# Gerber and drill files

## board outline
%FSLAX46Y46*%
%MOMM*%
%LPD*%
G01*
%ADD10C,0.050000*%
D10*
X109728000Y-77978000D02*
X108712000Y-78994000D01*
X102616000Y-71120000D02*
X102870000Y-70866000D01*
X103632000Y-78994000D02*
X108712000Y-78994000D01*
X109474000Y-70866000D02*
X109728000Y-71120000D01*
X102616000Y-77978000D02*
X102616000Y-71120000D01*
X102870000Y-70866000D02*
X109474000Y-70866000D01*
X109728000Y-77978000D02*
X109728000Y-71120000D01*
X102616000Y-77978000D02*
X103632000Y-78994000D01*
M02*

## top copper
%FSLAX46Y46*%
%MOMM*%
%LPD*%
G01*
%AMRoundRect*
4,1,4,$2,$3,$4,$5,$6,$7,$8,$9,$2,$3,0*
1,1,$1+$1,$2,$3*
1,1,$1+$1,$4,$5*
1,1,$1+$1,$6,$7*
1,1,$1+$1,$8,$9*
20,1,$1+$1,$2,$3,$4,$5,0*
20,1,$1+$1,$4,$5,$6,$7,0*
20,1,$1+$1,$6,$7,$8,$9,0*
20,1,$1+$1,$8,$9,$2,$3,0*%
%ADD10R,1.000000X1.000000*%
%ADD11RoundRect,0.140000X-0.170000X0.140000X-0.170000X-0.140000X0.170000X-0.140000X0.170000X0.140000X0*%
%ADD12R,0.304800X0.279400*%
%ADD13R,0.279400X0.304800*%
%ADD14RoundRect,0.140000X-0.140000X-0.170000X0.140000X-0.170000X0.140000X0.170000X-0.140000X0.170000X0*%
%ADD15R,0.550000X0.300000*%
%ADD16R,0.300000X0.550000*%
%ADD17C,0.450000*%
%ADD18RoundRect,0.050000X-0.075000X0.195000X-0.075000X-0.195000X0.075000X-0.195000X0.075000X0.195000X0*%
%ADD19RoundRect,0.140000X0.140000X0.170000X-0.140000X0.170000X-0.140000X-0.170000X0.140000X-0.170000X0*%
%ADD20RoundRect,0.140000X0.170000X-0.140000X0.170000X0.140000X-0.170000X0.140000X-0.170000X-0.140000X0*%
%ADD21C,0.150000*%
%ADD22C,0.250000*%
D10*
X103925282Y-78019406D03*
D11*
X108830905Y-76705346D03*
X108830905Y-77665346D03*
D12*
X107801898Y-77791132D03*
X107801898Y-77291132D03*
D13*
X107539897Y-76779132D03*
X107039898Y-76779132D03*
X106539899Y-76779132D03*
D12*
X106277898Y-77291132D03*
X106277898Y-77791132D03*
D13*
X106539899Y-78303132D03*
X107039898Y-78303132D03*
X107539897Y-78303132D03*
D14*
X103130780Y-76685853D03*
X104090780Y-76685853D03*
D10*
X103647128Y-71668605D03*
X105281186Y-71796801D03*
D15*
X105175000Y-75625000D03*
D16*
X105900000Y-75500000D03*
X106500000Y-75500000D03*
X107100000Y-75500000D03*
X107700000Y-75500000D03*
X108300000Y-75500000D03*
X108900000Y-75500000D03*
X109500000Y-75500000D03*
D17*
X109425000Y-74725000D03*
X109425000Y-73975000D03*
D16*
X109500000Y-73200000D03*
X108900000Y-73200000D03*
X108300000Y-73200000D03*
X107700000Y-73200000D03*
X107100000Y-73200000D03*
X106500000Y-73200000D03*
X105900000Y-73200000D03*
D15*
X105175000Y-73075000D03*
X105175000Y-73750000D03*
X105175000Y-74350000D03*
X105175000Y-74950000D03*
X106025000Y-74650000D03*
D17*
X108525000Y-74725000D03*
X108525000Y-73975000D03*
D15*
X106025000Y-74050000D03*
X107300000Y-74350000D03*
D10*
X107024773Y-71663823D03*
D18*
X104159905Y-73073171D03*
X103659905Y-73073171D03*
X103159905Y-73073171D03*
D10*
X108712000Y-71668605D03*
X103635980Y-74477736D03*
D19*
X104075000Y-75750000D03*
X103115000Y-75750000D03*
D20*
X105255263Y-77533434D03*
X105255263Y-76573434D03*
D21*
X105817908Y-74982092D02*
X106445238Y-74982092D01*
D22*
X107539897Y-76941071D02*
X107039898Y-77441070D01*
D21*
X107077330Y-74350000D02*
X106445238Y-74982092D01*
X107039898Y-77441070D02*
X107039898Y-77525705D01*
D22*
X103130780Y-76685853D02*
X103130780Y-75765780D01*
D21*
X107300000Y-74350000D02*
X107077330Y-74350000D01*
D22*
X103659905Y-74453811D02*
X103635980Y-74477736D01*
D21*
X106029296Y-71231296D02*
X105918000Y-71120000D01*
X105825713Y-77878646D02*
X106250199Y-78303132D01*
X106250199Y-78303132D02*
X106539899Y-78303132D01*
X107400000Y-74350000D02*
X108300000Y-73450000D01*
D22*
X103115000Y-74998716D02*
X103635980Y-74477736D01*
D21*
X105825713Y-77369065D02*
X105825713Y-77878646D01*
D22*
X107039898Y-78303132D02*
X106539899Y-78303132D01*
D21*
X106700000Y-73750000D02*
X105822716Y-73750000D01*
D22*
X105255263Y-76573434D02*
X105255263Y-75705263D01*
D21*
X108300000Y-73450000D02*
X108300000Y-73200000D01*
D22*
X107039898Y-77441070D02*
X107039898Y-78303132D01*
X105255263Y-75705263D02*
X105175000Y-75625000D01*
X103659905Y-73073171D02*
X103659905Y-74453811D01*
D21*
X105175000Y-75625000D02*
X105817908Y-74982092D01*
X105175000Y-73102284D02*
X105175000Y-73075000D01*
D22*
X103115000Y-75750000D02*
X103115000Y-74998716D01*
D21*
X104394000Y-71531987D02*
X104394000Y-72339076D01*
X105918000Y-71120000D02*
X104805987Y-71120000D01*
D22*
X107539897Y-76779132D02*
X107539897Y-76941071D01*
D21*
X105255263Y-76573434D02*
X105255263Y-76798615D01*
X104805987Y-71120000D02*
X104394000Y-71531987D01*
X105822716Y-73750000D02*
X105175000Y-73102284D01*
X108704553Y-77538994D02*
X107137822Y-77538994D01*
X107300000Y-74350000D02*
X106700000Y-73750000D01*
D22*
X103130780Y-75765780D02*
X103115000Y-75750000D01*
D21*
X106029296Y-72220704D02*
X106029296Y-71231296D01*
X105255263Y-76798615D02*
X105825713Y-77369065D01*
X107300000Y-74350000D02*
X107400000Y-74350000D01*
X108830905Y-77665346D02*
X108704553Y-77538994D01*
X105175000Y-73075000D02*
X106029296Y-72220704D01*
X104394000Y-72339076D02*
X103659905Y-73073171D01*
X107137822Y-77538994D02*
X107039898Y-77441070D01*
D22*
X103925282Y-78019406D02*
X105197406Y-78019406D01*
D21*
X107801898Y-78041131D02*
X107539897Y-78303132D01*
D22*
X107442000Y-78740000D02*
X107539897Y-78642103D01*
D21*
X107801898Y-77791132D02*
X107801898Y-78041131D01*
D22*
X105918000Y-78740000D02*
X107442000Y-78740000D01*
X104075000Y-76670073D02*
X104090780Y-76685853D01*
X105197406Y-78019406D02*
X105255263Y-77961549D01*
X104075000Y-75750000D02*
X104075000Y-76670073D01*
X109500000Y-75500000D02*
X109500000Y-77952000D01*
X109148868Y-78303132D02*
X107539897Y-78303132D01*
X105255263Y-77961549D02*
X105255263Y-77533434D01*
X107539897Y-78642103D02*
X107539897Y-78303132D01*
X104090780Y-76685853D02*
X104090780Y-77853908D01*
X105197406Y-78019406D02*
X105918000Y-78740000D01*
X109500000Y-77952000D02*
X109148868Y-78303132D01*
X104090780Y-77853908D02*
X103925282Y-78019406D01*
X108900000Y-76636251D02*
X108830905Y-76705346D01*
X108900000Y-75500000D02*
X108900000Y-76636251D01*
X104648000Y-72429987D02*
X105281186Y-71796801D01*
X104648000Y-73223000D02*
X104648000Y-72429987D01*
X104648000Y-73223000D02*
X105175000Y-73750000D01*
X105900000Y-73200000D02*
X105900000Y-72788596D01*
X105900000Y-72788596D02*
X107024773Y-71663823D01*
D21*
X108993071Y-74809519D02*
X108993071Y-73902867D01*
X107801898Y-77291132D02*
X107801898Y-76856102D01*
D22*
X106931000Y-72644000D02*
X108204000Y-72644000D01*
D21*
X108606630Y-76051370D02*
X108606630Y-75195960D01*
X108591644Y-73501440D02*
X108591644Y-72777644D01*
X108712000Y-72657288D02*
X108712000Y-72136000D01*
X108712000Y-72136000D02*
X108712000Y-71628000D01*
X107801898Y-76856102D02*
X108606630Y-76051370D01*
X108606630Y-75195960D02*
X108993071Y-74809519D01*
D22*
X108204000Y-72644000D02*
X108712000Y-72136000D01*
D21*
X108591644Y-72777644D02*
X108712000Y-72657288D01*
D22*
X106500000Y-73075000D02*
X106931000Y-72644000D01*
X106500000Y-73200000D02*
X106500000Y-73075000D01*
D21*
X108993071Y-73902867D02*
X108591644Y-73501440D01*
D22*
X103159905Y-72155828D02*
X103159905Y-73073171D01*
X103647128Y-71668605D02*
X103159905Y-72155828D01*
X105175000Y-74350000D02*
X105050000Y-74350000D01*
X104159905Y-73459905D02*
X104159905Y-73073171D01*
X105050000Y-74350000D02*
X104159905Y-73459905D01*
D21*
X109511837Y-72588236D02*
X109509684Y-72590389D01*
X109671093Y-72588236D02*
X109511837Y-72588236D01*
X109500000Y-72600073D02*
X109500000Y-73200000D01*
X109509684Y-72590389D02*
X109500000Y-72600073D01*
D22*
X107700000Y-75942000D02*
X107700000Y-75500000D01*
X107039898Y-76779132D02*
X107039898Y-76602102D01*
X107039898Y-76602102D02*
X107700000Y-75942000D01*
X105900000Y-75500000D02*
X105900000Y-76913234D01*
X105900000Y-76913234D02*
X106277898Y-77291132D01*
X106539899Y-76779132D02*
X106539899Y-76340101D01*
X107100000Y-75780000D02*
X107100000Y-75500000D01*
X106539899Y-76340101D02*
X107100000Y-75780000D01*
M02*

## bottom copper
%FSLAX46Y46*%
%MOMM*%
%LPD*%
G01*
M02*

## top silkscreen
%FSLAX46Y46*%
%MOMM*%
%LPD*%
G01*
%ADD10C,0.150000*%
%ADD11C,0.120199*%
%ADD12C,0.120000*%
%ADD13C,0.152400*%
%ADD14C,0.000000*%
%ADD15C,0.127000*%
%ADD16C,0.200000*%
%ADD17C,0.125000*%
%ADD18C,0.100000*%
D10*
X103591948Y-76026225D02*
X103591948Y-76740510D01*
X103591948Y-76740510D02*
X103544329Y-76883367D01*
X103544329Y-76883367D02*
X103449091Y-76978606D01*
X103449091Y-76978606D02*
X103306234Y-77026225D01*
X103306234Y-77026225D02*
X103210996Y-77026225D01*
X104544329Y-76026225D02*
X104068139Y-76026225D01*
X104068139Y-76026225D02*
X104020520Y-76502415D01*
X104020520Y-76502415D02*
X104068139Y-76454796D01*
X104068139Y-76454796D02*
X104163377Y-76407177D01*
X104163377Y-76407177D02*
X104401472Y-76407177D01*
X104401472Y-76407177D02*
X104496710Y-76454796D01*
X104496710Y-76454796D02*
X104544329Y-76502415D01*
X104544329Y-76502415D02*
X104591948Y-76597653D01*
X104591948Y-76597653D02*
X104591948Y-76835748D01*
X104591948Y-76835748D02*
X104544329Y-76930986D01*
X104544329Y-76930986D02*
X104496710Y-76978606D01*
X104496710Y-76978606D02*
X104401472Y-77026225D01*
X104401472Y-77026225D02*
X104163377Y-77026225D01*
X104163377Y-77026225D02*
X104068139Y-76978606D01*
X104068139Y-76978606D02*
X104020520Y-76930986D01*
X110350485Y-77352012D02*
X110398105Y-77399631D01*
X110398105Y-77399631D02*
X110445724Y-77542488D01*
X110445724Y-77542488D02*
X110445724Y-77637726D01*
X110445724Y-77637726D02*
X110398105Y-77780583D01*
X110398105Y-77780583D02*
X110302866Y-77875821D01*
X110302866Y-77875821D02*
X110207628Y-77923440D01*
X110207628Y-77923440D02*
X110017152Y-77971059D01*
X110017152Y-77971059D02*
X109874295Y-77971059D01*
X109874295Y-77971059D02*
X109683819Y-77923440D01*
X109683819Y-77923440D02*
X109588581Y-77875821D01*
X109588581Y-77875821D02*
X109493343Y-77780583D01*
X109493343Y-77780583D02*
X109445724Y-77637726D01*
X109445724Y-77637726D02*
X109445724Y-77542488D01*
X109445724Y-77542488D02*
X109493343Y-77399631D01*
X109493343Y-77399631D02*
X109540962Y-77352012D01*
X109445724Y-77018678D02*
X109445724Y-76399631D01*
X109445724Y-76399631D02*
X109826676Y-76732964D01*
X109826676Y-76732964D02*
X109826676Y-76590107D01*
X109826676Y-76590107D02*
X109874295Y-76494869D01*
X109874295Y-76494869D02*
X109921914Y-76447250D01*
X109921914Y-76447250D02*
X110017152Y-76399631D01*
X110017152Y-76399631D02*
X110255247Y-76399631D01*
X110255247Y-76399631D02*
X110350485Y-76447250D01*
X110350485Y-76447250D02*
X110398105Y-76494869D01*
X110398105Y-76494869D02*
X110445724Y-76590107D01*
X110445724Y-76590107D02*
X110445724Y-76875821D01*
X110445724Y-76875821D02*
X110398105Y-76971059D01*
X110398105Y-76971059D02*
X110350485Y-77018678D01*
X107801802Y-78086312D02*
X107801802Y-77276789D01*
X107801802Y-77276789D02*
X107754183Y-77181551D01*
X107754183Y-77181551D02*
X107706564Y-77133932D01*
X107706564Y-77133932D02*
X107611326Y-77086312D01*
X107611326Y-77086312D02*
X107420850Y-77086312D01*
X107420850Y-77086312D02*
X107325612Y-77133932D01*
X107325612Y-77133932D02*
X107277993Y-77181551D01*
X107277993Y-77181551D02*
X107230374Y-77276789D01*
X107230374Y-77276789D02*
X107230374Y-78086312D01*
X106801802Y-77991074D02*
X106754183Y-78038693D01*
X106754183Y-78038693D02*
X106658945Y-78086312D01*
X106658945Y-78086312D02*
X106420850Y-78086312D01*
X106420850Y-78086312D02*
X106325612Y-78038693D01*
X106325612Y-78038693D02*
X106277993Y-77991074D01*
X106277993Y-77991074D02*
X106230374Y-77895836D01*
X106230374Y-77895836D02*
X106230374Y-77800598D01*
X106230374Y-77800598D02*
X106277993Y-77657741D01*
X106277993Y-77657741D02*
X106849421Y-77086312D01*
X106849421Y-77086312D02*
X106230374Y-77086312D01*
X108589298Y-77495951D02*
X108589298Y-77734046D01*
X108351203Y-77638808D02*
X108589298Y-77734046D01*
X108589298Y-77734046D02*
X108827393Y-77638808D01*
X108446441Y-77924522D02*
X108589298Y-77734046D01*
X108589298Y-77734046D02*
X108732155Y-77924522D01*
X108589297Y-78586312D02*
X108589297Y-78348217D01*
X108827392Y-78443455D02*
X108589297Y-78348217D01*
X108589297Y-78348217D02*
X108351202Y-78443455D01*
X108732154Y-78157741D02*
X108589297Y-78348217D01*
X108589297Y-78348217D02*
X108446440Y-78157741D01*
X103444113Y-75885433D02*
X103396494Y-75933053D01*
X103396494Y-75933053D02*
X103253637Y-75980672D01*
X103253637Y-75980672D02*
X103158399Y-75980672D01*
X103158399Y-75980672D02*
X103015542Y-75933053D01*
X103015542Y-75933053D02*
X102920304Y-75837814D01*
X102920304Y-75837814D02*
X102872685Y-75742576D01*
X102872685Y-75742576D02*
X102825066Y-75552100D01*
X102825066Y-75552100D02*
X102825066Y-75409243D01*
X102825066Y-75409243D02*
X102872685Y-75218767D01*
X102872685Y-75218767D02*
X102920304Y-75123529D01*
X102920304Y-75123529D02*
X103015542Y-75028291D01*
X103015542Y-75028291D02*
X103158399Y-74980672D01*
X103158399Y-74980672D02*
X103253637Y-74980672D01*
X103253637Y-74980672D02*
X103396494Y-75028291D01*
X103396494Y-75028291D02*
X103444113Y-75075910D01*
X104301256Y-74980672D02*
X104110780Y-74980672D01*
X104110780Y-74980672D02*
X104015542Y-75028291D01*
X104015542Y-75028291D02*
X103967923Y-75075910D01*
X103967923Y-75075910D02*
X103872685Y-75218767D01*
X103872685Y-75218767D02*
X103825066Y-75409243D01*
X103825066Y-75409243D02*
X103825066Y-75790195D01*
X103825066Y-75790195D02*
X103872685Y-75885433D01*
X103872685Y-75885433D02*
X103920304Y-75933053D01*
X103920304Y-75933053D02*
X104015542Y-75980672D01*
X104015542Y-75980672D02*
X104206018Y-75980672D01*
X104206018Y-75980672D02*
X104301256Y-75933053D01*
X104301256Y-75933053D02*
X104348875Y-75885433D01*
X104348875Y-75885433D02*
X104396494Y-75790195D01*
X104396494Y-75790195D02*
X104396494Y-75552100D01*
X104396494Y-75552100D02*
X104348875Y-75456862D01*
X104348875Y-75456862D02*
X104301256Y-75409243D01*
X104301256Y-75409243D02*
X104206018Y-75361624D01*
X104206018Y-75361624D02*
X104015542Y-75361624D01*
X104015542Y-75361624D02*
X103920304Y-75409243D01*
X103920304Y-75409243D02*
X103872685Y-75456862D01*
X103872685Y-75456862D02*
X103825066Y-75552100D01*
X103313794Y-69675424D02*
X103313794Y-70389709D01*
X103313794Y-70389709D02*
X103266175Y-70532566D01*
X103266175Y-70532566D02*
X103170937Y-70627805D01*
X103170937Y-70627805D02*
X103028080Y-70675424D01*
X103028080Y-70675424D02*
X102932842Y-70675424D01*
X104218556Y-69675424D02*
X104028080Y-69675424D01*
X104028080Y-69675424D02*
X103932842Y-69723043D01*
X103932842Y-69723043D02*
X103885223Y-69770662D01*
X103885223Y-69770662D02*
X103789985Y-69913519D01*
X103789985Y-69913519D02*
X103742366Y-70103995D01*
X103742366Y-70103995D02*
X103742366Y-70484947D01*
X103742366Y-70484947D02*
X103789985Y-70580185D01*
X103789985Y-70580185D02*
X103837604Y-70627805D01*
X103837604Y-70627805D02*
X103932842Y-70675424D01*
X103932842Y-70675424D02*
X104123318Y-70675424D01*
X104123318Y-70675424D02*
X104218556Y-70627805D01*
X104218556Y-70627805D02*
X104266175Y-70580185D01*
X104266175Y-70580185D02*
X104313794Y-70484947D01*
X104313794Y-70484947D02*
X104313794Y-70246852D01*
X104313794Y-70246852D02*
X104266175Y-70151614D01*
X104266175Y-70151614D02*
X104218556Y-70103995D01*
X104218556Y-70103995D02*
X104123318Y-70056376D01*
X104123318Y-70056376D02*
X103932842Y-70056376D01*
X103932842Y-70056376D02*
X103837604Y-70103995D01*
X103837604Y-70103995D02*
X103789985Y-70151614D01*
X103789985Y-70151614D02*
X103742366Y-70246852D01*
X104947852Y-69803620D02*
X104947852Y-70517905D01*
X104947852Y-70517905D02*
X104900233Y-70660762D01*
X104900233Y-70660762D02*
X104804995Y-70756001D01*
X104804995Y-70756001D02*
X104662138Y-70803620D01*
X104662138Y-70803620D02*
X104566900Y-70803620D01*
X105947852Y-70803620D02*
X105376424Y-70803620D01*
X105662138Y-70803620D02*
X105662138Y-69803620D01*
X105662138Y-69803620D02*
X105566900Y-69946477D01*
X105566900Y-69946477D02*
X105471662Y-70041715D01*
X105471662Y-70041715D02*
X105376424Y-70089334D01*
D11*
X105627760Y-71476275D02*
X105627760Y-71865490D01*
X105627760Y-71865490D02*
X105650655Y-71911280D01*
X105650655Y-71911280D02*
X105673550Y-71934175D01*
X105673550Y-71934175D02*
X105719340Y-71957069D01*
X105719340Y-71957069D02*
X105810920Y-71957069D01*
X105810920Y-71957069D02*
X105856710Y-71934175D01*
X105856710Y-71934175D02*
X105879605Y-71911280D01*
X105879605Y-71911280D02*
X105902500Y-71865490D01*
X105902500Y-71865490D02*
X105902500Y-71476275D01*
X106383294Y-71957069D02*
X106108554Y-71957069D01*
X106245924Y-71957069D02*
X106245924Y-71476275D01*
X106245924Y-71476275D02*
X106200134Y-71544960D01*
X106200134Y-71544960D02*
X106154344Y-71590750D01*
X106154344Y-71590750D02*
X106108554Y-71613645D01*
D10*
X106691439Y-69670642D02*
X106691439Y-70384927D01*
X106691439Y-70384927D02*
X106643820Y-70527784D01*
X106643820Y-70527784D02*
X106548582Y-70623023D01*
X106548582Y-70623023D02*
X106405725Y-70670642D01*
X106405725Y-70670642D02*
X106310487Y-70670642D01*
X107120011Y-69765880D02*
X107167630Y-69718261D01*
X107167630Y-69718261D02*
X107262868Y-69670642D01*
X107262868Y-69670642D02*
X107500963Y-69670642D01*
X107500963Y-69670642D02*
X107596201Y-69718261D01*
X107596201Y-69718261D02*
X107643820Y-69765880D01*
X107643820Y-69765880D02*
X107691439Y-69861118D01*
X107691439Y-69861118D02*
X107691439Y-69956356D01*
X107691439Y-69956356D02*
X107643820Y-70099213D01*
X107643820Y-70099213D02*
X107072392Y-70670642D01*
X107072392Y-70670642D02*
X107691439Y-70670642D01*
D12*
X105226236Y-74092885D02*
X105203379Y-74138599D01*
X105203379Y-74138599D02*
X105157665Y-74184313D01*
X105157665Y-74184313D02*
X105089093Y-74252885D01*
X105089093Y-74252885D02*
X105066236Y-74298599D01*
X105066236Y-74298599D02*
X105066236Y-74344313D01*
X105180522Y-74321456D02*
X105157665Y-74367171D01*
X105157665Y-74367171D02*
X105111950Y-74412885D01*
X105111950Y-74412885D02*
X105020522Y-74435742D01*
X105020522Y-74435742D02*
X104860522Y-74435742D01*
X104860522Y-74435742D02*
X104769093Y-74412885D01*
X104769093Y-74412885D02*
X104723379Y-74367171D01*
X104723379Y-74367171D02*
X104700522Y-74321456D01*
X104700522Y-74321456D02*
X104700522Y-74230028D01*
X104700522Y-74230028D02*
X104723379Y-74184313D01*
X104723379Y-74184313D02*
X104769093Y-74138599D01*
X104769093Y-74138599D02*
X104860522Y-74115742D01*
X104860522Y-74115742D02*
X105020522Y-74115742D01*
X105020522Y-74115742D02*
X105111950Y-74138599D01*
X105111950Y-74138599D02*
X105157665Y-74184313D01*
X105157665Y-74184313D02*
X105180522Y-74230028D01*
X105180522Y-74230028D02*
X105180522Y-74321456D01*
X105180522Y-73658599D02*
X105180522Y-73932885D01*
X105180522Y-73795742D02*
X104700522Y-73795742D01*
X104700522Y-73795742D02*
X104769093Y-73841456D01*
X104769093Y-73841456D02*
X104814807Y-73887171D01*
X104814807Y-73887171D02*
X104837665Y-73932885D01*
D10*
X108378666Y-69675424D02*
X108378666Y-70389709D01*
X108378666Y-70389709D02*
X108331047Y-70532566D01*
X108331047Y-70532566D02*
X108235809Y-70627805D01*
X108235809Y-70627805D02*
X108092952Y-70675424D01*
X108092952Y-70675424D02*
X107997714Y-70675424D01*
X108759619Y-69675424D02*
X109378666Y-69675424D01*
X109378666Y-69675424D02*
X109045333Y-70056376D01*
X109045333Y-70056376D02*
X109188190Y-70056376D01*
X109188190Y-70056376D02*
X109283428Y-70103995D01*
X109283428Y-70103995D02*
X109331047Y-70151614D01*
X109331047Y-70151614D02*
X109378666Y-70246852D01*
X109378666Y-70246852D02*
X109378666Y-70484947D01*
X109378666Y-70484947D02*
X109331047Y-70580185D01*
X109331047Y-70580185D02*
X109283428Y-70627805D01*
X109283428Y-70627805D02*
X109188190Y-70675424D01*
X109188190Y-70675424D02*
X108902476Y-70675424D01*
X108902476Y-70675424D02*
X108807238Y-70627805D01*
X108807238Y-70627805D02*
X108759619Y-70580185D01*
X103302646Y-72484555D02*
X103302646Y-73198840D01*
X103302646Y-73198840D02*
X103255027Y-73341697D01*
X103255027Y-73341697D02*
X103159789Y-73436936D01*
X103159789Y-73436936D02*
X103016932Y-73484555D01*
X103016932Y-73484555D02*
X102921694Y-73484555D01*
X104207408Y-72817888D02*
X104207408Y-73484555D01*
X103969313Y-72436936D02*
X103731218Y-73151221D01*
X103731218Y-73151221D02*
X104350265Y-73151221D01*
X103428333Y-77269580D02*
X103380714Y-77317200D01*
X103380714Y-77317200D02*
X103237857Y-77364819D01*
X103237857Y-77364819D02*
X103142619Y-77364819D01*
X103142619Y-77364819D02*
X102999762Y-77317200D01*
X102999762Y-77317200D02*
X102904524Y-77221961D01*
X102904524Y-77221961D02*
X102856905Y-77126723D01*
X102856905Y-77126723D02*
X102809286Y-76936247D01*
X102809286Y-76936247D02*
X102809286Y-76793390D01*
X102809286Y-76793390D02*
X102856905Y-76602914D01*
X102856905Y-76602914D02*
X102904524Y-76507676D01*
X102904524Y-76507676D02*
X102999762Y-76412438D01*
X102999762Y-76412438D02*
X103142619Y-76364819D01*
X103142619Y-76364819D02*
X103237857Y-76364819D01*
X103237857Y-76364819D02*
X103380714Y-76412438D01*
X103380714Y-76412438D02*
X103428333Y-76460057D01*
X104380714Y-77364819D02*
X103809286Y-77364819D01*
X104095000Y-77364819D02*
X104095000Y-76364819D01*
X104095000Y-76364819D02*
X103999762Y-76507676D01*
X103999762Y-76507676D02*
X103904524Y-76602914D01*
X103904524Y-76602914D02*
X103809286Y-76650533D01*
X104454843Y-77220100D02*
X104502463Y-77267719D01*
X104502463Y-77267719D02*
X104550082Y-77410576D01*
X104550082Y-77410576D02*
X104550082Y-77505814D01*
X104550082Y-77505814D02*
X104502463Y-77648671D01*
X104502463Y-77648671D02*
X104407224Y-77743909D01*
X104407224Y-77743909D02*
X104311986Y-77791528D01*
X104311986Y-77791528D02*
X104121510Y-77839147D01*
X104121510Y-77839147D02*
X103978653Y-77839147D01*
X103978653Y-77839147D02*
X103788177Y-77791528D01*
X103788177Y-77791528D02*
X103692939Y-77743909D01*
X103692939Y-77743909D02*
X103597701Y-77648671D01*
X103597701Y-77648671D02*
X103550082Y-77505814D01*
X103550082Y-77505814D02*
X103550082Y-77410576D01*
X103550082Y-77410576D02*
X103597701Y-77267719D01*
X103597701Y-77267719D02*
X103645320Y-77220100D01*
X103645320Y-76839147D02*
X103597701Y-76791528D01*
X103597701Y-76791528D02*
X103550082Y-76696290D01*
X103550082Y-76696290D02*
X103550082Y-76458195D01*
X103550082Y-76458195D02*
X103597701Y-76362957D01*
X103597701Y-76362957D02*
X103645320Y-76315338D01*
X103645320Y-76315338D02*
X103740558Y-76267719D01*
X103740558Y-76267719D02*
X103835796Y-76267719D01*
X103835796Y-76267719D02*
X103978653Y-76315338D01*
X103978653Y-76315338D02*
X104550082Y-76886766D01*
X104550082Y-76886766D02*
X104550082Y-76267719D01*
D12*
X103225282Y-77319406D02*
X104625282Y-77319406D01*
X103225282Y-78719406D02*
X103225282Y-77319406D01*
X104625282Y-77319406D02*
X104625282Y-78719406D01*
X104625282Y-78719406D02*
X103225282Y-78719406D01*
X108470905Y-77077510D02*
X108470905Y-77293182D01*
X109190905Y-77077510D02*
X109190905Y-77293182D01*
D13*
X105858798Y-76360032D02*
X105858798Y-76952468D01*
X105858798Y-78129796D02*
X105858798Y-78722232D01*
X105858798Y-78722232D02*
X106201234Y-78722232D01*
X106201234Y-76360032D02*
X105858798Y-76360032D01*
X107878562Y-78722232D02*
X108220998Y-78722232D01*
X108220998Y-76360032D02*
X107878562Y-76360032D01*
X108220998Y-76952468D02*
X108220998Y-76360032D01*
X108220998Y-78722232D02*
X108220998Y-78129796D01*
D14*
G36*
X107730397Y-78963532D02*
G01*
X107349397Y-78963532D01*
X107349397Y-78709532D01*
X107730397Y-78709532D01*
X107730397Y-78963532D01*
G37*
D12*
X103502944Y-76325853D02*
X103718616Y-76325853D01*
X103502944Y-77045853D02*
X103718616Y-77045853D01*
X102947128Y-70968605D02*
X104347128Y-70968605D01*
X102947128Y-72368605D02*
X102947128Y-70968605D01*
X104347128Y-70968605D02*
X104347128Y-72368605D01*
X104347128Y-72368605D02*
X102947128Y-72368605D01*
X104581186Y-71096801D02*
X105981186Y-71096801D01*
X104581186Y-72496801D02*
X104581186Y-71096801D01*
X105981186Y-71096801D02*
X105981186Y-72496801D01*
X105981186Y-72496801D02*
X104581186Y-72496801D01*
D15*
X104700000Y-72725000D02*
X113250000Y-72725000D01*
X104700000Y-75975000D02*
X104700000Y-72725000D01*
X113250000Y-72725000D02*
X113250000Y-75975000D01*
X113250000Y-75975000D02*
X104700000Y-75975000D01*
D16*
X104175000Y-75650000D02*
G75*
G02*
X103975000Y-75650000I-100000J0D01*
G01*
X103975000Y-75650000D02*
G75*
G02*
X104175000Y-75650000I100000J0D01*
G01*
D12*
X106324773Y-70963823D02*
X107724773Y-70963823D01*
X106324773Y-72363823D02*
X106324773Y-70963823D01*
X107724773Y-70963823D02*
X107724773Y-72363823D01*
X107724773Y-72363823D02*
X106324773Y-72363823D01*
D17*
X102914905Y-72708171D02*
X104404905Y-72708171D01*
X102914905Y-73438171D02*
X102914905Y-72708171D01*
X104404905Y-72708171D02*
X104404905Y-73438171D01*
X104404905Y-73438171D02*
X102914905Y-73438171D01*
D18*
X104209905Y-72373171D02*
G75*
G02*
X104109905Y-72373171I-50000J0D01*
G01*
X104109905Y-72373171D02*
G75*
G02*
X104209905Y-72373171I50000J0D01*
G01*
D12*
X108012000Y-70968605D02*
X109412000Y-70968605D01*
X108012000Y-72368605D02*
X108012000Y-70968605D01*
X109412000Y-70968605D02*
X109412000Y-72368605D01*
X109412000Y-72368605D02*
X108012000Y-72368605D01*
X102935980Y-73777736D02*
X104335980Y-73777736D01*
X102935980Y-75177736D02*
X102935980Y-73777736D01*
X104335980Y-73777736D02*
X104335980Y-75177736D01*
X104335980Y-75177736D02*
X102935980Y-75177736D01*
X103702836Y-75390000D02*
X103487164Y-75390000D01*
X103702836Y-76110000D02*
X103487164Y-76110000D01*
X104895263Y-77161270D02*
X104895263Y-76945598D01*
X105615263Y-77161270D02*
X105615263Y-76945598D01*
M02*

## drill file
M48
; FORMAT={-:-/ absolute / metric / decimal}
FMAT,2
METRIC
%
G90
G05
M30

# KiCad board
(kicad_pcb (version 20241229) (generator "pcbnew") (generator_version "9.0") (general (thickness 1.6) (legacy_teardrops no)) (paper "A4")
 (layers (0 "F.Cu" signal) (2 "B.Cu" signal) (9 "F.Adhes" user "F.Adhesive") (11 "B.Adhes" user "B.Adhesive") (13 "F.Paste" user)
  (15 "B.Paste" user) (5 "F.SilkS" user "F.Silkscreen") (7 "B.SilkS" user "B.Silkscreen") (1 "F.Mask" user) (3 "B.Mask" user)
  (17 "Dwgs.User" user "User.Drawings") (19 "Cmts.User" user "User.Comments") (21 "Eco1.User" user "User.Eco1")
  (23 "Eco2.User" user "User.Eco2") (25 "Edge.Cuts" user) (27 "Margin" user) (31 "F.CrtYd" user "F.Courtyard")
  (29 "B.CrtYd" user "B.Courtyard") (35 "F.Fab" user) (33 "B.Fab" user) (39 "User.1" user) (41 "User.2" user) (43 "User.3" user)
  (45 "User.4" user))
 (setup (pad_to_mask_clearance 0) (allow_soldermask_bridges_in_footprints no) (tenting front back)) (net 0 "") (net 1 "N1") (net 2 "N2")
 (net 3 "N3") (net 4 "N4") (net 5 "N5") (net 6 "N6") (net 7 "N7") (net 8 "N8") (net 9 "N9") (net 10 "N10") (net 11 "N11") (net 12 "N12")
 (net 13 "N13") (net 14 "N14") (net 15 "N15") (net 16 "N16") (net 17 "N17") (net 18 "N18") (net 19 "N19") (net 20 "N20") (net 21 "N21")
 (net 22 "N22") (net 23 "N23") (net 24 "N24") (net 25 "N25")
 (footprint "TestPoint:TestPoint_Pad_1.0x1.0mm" (layer "F.Cu") (at 103.925282 78.019406)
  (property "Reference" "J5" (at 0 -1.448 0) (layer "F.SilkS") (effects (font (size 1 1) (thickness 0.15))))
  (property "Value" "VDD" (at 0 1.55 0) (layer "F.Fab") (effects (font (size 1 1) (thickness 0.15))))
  (fp_line (start -0.7 -0.7) (end 0.7 -0.7) (stroke (width 0.12) (type solid)) (layer "F.SilkS"))
  (fp_line (start -0.7 0.7) (end -0.7 -0.7) (stroke (width 0.12) (type solid)) (layer "F.SilkS"))
  (fp_line (start 0.7 -0.7) (end 0.7 0.7) (stroke (width 0.12) (type solid)) (layer "F.SilkS"))
  (fp_line (start 0.7 0.7) (end -0.7 0.7) (stroke (width 0.12) (type solid)) (layer "F.SilkS"))
  (pad "1" smd rect (at 0 0) (size 1 1) (layers "F.Cu" "F.Mask") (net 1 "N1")))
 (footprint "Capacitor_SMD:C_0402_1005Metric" (layer "F.Cu") (at 108.830905 77.185346 -90)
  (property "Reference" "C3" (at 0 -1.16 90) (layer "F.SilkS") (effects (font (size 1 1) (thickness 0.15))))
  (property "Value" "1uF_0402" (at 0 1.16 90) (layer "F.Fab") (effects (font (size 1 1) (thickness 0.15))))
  (fp_line (start -0.107836 0.36) (end 0.107836 0.36) (stroke (width 0.12) (type solid)) (layer "F.SilkS"))
  (fp_line (start -0.107836 -0.36) (end 0.107836 -0.36) (stroke (width 0.12) (type solid)) (layer "F.SilkS"))
  (pad "1" smd roundrect (at -0.48 0 270) (size 0.56 0.62) (layers "F.Cu" "F.Mask" "F.Paste") (roundrect_rratio 0.25) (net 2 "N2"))
  (pad "2" smd roundrect (at 0.48 0 270) (size 0.56 0.62) (layers "F.Cu" "F.Mask" "F.Paste") (roundrect_rratio 0.25) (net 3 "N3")))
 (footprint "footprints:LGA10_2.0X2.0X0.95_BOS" (layer "F.Cu") (at 107.039898 77.541132 180)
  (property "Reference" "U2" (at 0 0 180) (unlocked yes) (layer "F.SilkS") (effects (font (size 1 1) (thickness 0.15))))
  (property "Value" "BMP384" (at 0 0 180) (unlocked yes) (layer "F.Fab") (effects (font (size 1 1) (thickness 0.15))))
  (fp_line (start 1.1811 1.1811) (end 1.1811 0.588664) (stroke (width 0.1524) (type solid)) (layer "F.SilkS"))
  (fp_line (start 1.1811 -0.588664) (end 1.1811 -1.1811) (stroke (width 0.1524) (type solid)) (layer "F.SilkS"))
  (fp_line (start 1.1811 -1.1811) (end 0.838664 -1.1811) (stroke (width 0.1524) (type solid)) (layer "F.SilkS"))
  (fp_line (start 0.838664 1.1811) (end 1.1811 1.1811) (stroke (width 0.1524) (type solid)) (layer "F.SilkS"))
  (fp_line (start -0.838664 -1.1811) (end -1.1811 -1.1811) (stroke (width 0.1524) (type solid)) (layer "F.SilkS"))
  (fp_line (start -1.1811 1.1811) (end -0.838664 1.1811) (stroke (width 0.1524) (type solid)) (layer "F.SilkS"))
  (fp_line (start -1.1811 0.588664) (end -1.1811 1.1811) (stroke (width 0.1524) (type solid)) (layer "F.SilkS"))
  (fp_line (start -1.1811 -1.1811) (end -1.1811 -0.588664) (stroke (width 0.1524) (type solid)) (layer "F.SilkS"))
  (fp_poly
   (pts (xy -0.690499 -1.1684) (xy -0.690499 -1.4224) (xy -0.309499 -1.4224) (xy -0.309499 -1.1684)) (stroke (width 0) (type solid))
   (fill yes) (layer "F.SilkS"))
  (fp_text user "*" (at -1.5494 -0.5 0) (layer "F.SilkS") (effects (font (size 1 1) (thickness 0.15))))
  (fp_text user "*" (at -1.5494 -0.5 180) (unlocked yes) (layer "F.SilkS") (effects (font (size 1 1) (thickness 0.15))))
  (pad "1" smd rect (at -0.762 -0.25 270) (size 0.2794 0.3048) (layers "F.Cu" "F.Mask" "F.Paste") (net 1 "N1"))
  (pad "2" smd rect (at -0.762 0.25 270) (size 0.2794 0.3048) (layers "F.Cu" "F.Mask" "F.Paste") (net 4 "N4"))
  (pad "3" smd rect (at -0.499999 0.762 180) (size 0.2794 0.3048) (layers "F.Cu" "F.Mask" "F.Paste") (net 3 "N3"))
  (pad "4" smd rect (at 0 0.762 180) (size 0.2794 0.3048) (layers "F.Cu" "F.Mask" "F.Paste") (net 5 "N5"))
  (pad "5" smd rect (at 0.499999 0.762 180) (size 0.2794 0.3048) (layers "F.Cu" "F.Mask" "F.Paste") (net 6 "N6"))
  (pad "6" smd rect (at 0.762 0.25 270) (size 0.2794 0.3048) (layers "F.Cu" "F.Mask" "F.Paste") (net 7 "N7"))
  (pad "7" smd rect (at 0.762 -0.25 270) (size 0.2794 0.3048) (layers "F.Cu" "F.Mask" "F.Paste") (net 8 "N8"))
  (pad "8" smd rect (at 0.499999 -0.762 180) (size 0.2794 0.3048) (layers "F.Cu" "F.Mask" "F.Paste") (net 3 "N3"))
  (pad "9" smd rect (at 0 -0.762 180) (size 0.2794 0.3048) (layers "F.Cu" "F.Mask" "F.Paste") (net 3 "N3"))
  (pad "10" smd rect (at -0.499999 -0.762 180) (size 0.2794 0.3048) (layers "F.Cu" "F.Mask" "F.Paste") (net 1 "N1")))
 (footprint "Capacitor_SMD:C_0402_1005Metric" (layer "F.Cu") (at 103.61078 76.685853)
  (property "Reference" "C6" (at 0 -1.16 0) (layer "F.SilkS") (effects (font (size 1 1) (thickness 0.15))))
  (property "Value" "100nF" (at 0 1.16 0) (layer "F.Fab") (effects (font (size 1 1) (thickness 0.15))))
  (fp_line (start -0.107836 -0.36) (end 0.107836 -0.36) (stroke (width 0.12) (type solid)) (layer "F.SilkS"))
  (fp_line (start -0.107836 0.36) (end 0.107836 0.36) (stroke (width 0.12) (type solid)) (layer "F.SilkS"))
  (pad "1" smd roundrect (at -0.48 0) (size 0.56 0.62) (layers "F.Cu" "F.Mask" "F.Paste") (roundrect_rratio 0.25) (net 3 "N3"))
  (pad "2" smd roundrect (at 0.48 0) (size 0.56 0.62) (layers "F.Cu" "F.Mask" "F.Paste") (roundrect_rratio 0.25) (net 1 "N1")))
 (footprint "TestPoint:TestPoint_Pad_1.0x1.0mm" (layer "F.Cu") (at 103.647128 71.668605)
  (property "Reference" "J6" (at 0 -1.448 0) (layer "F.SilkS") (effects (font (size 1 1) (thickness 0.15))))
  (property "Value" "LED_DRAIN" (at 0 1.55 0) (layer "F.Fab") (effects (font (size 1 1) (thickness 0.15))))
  (fp_line (start -0.7 -0.7) (end 0.7 -0.7) (stroke (width 0.12) (type solid)) (layer "F.SilkS"))
  (fp_line (start -0.7 0.7) (end -0.7 -0.7) (stroke (width 0.12) (type solid)) (layer "F.SilkS"))
  (fp_line (start 0.7 -0.7) (end 0.7 0.7) (stroke (width 0.12) (type solid)) (layer "F.SilkS"))
  (fp_line (start 0.7 0.7) (end -0.7 0.7) (stroke (width 0.12) (type solid)) (layer "F.SilkS"))
  (pad "1" smd rect (at 0 0) (size 1 1) (layers "F.Cu" "F.Mask") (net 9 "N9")))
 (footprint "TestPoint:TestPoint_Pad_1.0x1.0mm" (layer "F.Cu") (at 105.281186 71.796801)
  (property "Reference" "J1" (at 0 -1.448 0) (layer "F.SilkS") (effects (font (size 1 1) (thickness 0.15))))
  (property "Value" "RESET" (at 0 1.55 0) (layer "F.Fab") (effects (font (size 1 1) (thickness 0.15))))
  (fp_line (start -0.7 -0.7) (end 0.7 -0.7) (stroke (width 0.12) (type solid)) (layer "F.SilkS"))
  (fp_line (start -0.7 0.7) (end -0.7 -0.7) (stroke (width 0.12) (type solid)) (layer "F.SilkS"))
  (fp_line (start 0.7 -0.7) (end 0.7 0.7) (stroke (width 0.12) (type solid)) (layer "F.SilkS"))
  (fp_line (start 0.7 0.7) (end -0.7 0.7) (stroke (width 0.12) (type solid)) (layer "F.SilkS"))
  (pad "1" smd rect (at 0 0) (size 1 1) (layers "F.Cu" "F.Mask") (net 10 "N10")))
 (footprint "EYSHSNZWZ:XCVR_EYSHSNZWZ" (layer "F.Cu") (at 108.975 74.35)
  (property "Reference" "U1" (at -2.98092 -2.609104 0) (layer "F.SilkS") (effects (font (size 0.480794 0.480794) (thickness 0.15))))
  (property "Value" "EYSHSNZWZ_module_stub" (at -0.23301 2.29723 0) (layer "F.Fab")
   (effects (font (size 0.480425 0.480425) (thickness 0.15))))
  (fp_line (start -4.275 -1.625) (end 4.275 -1.625) (stroke (width 0.127) (type solid)) (layer "F.SilkS"))
  (fp_line (start -4.275 1.625) (end -4.275 -1.625) (stroke (width 0.127) (type solid)) (layer "F.SilkS"))
  (fp_line (start 4.275 -1.625) (end 4.275 1.625) (stroke (width 0.127) (type solid)) (layer "F.SilkS"))
  (fp_line (start 4.275 1.625) (end -4.275 1.625) (stroke (width 0.127) (type solid)) (layer "F.SilkS"))
  (fp_circle (center -4.9 1.3) (end -4.8 1.3) (stroke (width 0.2) (type solid)) (fill no) (layer "F.SilkS"))
  (pad "1" smd rect (at -3.8 1.275) (size 0.55 0.3) (layers "F.Cu" "F.Mask") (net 3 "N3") (solder_mask_margin 0.102))
  (pad "2" smd rect (at -3.075 1.15) (size 0.3 0.55) (layers "F.Cu" "F.Mask") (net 7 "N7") (solder_mask_margin 0.102))
  (pad "3" smd rect (at -2.475 1.15) (size 0.3 0.55) (layers "F.Cu" "F.Mask") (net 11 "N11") (solder_mask_margin 0.102))
  (pad "4" smd rect (at -1.875 1.15) (size 0.3 0.55) (layers "F.Cu" "F.Mask") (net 6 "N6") (solder_mask_margin 0.102))
  (pad "5" smd rect (at -1.275 1.15) (size 0.3 0.55) (layers "F.Cu" "F.Mask") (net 5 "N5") (solder_mask_margin 0.102))
  (pad "6" smd rect (at -0.675 1.15) (size 0.3 0.55) (layers "F.Cu" "F.Mask") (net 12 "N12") (solder_mask_margin 0.102))
  (pad "7" smd rect (at -0.075 1.15) (size 0.3 0.55) (layers "F.Cu" "F.Mask") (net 2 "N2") (solder_mask_margin 0.102))
  (pad "8" smd rect (at 0.525 1.15) (size 0.3 0.55) (layers "F.Cu" "F.Mask") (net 1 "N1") (solder_mask_margin 0.102))
  (pad "9" smd circle (at 0.45 0.375) (size 0.45 0.45) (layers "F.Cu" "F.Mask") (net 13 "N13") (solder_mask_margin 0.102))
  (pad "10" smd circle (at 0.45 -0.375) (size 0.45 0.45) (layers "F.Cu" "F.Mask") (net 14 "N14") (solder_mask_margin 0.102))
  (pad "11" smd rect (at 0.525 -1.15) (size 0.3 0.55) (layers "F.Cu" "F.Mask") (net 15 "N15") (solder_mask_margin 0.102))
  (pad "12" smd rect (at -0.075 -1.15) (size 0.3 0.55) (layers "F.Cu" "F.Mask") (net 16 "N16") (solder_mask_margin 0.102))
  (pad "13" smd rect (at -0.675 -1.15) (size 0.3 0.55) (layers "F.Cu" "F.Mask") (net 3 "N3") (solder_mask_margin 0.102))
  (pad "14" smd rect (at -1.275 -1.15) (size 0.3 0.55) (layers "F.Cu" "F.Mask") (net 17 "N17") (solder_mask_margin 0.102))
  (pad "15" smd rect (at -1.875 -1.15) (size 0.3 0.55) (layers "F.Cu" "F.Mask") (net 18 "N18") (solder_mask_margin 0.102))
  (pad "16" smd rect (at -2.475 -1.15) (size 0.3 0.55) (layers "F.Cu" "F.Mask") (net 4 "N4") (solder_mask_margin 0.102))
  (pad "17" smd rect (at -3.075 -1.15) (size 0.3 0.55) (layers "F.Cu" "F.Mask") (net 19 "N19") (solder_mask_margin 0.102))
  (pad "18" smd rect (at -3.8 -1.275) (size 0.55 0.3) (layers "F.Cu" "F.Mask") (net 3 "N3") (solder_mask_margin 0.102))
  (pad "19" smd rect (at -3.8 -0.6) (size 0.55 0.3) (layers "F.Cu" "F.Mask") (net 10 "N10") (solder_mask_margin 0.102))
  (pad "20" smd rect (at -3.8 0) (size 0.55 0.3) (layers "F.Cu" "F.Mask") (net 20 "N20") (solder_mask_margin 0.102))
  (pad "21" smd rect (at -3.8 0.6) (size 0.55 0.3) (layers "F.Cu" "F.Mask") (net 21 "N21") (solder_mask_margin 0.102))
  (pad "22" smd rect (at -2.95 0.3) (size 0.55 0.3) (layers "F.Cu" "F.Mask") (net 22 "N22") (solder_mask_margin 0.102))
  (pad "23" smd circle (at -0.45 0.375) (size 0.45 0.45) (layers "F.Cu" "F.Mask") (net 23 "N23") (solder_mask_margin 0.102))
  (pad "24" smd circle (at -0.45 -0.375) (size 0.45 0.45) (layers "F.Cu" "F.Mask") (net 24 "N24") (solder_mask_margin 0.102))
  (pad "25" smd rect (at -2.95 -0.3) (size 0.55 0.3) (layers "F.Cu" "F.Mask") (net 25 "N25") (solder_mask_margin 0.102))
  (pad "26" smd rect (at -1.675 0) (size 0.55 0.3) (layers "F.Cu" "F.Mask") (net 3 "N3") (solder_mask_margin 0.102)))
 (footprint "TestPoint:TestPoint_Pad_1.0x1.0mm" (layer "F.Cu") (at 107.024773 71.663823)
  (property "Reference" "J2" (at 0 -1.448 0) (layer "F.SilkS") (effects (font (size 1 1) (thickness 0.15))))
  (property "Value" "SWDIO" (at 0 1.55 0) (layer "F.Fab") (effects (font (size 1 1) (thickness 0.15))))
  (fp_line (start -0.7 -0.7) (end 0.7 -0.7) (stroke (width 0.12) (type solid)) (layer "F.SilkS"))
  (fp_line (start -0.7 0.7) (end -0.7 -0.7) (stroke (width 0.12) (type solid)) (layer "F.SilkS"))
  (fp_line (start 0.7 -0.7) (end 0.7 0.7) (stroke (width 0.12) (type solid)) (layer "F.SilkS"))
  (fp_line (start 0.7 0.7) (end -0.7 0.7) (stroke (width 0.12) (type solid)) (layer "F.SilkS"))
  (pad "1" smd rect (at 0 0) (size 1 1) (layers "F.Cu" "F.Mask") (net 19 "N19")))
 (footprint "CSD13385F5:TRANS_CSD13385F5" (layer "F.Cu") (at 103.659905 73.073171 -90)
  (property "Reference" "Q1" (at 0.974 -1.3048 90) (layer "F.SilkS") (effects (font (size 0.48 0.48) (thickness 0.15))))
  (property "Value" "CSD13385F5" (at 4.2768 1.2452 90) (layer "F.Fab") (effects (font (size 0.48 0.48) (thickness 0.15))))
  (fp_line (start -0.365 0.745) (end -0.365 -0.745) (stroke (width 0.125) (type solid)) (layer "F.SilkS"))
  (fp_line (start 0.365 0.745) (end -0.365 0.745) (stroke (width 0.125) (type solid)) (layer "F.SilkS"))
  (fp_line (start -0.365 -0.745) (end 0.365 -0.745) (stroke (width 0.125) (type solid)) (layer "F.SilkS"))
  (fp_line (start 0.365 -0.745) (end 0.365 0.745) (stroke (width 0.125) (type solid)) (layer "F.SilkS"))
  (fp_circle (center -0.7 -0.5) (end -0.65 -0.5) (stroke (width 0.1) (type solid)) (fill no) (layer "F.SilkS"))
  (pad "1" smd roundrect (at 0 -0.5 270) (size 0.49 0.25) (layers "F.Cu") (roundrect_rratio 0.2) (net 20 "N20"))
  (pad "2" smd roundrect (at 0 0 270) (size 0.49 0.25) (layers "F.Cu") (roundrect_rratio 0.2) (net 3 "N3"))
  (pad "3" smd roundrect (at 0 0.5 270) (size 0.49 0.25) (layers "F.Cu") (roundrect_rratio 0.2) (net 9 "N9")))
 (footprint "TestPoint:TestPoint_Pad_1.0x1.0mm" (layer "F.Cu") (at 108.712 71.668605)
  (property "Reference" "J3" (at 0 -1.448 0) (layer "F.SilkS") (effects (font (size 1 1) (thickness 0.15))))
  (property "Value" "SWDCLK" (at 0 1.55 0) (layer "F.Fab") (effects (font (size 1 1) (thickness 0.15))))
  (fp_line (start -0.7 -0.7) (end 0.7 -0.7) (stroke (width 0.12) (type solid)) (layer "F.SilkS"))
  (fp_line (start -0.7 0.7) (end -0.7 -0.7) (stroke (width 0.12) (type solid)) (layer "F.SilkS"))
  (fp_line (start 0.7 -0.7) (end 0.7 0.7) (stroke (width 0.12) (type solid)) (layer "F.SilkS"))
  (fp_line (start 0.7 0.7) (end -0.7 0.7) (stroke (width 0.12) (type solid)) (layer "F.SilkS"))
  (pad "1" smd rect (at 0 0) (size 1 1) (layers "F.Cu" "F.Mask") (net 4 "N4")))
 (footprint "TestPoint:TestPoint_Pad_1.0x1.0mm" (layer "F.Cu") (at 103.63598 74.477736)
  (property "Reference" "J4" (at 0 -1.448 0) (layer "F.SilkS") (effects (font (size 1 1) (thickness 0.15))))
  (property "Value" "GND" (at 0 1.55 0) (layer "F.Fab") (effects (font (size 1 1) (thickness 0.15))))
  (fp_line (start -0.7 -0.7) (end 0.7 -0.7) (stroke (width 0.12) (type solid)) (layer "F.SilkS"))
  (fp_line (start -0.7 0.7) (end -0.7 -0.7) (stroke (width 0.12) (type solid)) (layer "F.SilkS"))
  (fp_line (start 0.7 -0.7) (end 0.7 0.7) (stroke (width 0.12) (type solid)) (layer "F.SilkS"))
  (fp_line (start 0.7 0.7) (end -0.7 0.7) (stroke (width 0.12) (type solid)) (layer "F.SilkS"))
  (pad "1" smd rect (at 0 0) (size 1 1) (layers "F.Cu" "F.Mask") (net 3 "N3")))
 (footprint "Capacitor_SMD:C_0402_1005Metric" (layer "F.Cu") (at 103.595 75.75 180)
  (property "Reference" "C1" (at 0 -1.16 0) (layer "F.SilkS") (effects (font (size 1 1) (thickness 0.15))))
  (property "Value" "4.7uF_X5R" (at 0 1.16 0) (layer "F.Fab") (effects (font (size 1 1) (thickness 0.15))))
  (fp_line (start -0.107836 0.36) (end 0.107836 0.36) (stroke (width 0.12) (type solid)) (layer "F.SilkS"))
  (fp_line (start -0.107836 -0.36) (end 0.107836 -0.36) (stroke (width 0.12) (type solid)) (layer "F.SilkS"))
  (pad "1" smd roundrect (at -0.48 0 180) (size 0.56 0.62) (layers "F.Cu" "F.Mask" "F.Paste") (roundrect_rratio 0.25) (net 1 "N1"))
  (pad "2" smd roundrect (at 0.48 0 180) (size 0.56 0.62) (layers "F.Cu" "F.Mask" "F.Paste") (roundrect_rratio 0.25) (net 3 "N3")))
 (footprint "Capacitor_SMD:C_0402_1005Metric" (layer "F.Cu") (at 105.255263 77.053434 90)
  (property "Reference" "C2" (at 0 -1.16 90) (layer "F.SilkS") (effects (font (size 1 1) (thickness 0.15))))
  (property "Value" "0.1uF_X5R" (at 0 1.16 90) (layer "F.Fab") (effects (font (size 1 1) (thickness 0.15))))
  (fp_line (start -0.107836 -0.36) (end 0.107836 -0.36) (stroke (width 0.12) (type solid)) (layer "F.SilkS"))
  (fp_line (start -0.107836 0.36) (end 0.107836 0.36) (stroke (width 0.12) (type solid)) (layer "F.SilkS"))
  (pad "1" smd roundrect (at -0.48 0 90) (size 0.56 0.62) (layers "F.Cu" "F.Mask" "F.Paste") (roundrect_rratio 0.25) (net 1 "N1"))
  (pad "2" smd roundrect (at 0.48 0 90) (size 0.56 0.62) (layers "F.Cu" "F.Mask" "F.Paste") (roundrect_rratio 0.25) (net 3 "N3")))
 (gr_line (start 109.728 77.978) (end 108.712 78.994) (stroke (width 0.05) (type default)) (layer "Edge.Cuts"))
 (gr_line (start 102.616 71.12) (end 102.87 70.866) (stroke (width 0.05) (type default)) (layer "Edge.Cuts"))
 (gr_line (start 103.632 78.994) (end 108.712 78.994) (stroke (width 0.05) (type default)) (layer "Edge.Cuts"))
 (gr_line (start 109.474 70.866) (end 109.728 71.12) (stroke (width 0.05) (type default)) (layer "Edge.Cuts"))
 (gr_line (start 102.616 77.978) (end 102.616 71.12) (stroke (width 0.05) (type default)) (layer "Edge.Cuts"))
 (gr_line (start 102.87 70.866) (end 109.474 70.866) (stroke (width 0.05) (type default)) (layer "Edge.Cuts"))
 (gr_line (start 109.728 77.978) (end 109.728 71.12) (stroke (width 0.05) (type default)) (layer "Edge.Cuts"))
 (gr_line (start 102.616 77.978) (end 103.632 78.994) (stroke (width 0.05) (type default)) (layer "Edge.Cuts"))
 (segment (start 105.817908 74.982092) (end 106.445238 74.982092) (width 0.15) (layer "F.Cu") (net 3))
 (segment (start 107.539897 76.941071) (end 107.039898 77.44107) (width 0.25) (layer "F.Cu") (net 3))
 (segment (start 107.07733 74.35) (end 106.445238 74.982092) (width 0.15) (layer "F.Cu") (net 3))
 (segment (start 107.039898 77.44107) (end 107.039898 77.525705) (width 0.15) (layer "F.Cu") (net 3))
 (segment (start 103.13078 76.685853) (end 103.13078 75.76578) (width 0.25) (layer "F.Cu") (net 3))
 (segment (start 107.3 74.35) (end 107.07733 74.35) (width 0.15) (layer "F.Cu") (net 3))
 (segment (start 103.659905 74.453811) (end 103.63598 74.477736) (width 0.25) (layer "F.Cu") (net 3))
 (segment (start 106.029296 71.231296) (end 105.918 71.12) (width 0.15) (layer "F.Cu") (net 3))
 (segment (start 105.825713 77.878646) (end 106.250199 78.303132) (width 0.15) (layer "F.Cu") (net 3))
 (segment (start 106.250199 78.303132) (end 106.539899 78.303132) (width 0.15) (layer "F.Cu") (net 3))
 (segment (start 107.4 74.35) (end 108.3 73.45) (width 0.15) (layer "F.Cu") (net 3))
 (segment (start 103.115 74.998716) (end 103.63598 74.477736) (width 0.25) (layer "F.Cu") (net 3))
 (segment (start 105.825713 77.369065) (end 105.825713 77.878646) (width 0.15) (layer "F.Cu") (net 3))
 (segment (start 107.039898 78.303132) (end 106.539899 78.303132) (width 0.25) (layer "F.Cu") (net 3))
 (segment (start 106.7 73.75) (end 105.822716 73.75) (width 0.15) (layer "F.Cu") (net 3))
 (segment (start 105.255263 76.573434) (end 105.255263 75.705263) (width 0.25) (layer "F.Cu") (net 3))
 (segment (start 108.3 73.45) (end 108.3 73.2) (width 0.15) (layer "F.Cu") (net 3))
 (segment (start 107.039898 77.44107) (end 107.039898 78.303132) (width 0.25) (layer "F.Cu") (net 3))
 (segment (start 105.255263 75.705263) (end 105.175 75.625) (width 0.25) (layer "F.Cu") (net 3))
 (segment (start 103.659905 73.073171) (end 103.659905 74.453811) (width 0.25) (layer "F.Cu") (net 3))
 (segment (start 105.175 75.625) (end 105.817908 74.982092) (width 0.15) (layer "F.Cu") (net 3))
 (segment (start 105.175 73.102284) (end 105.175 73.075) (width 0.15) (layer "F.Cu") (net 3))
 (segment (start 103.115 75.75) (end 103.115 74.998716) (width 0.25) (layer "F.Cu") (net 3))
 (segment (start 104.394 71.531987) (end 104.394 72.339076) (width 0.15) (layer "F.Cu") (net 3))
 (segment (start 105.918 71.12) (end 104.805987 71.12) (width 0.15) (layer "F.Cu") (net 3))
 (segment (start 107.539897 76.779132) (end 107.539897 76.941071) (width 0.25) (layer "F.Cu") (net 3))
 (segment (start 105.255263 76.573434) (end 105.255263 76.798615) (width 0.15) (layer "F.Cu") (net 3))
 (segment (start 104.805987 71.12) (end 104.394 71.531987) (width 0.15) (layer "F.Cu") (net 3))
 (segment (start 105.822716 73.75) (end 105.175 73.102284) (width 0.15) (layer "F.Cu") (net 3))
 (segment (start 108.704553 77.538994) (end 107.137822 77.538994) (width 0.15) (layer "F.Cu") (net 3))
 (segment (start 107.3 74.35) (end 106.7 73.75) (width 0.15) (layer "F.Cu") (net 3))
 (segment (start 103.13078 75.76578) (end 103.115 75.75) (width 0.25) (layer "F.Cu") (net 3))
 (segment (start 106.029296 72.220704) (end 106.029296 71.231296) (width 0.15) (layer "F.Cu") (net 3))
 (segment (start 105.255263 76.798615) (end 105.825713 77.369065) (width 0.15) (layer "F.Cu") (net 3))
 (segment (start 107.3 74.35) (end 107.4 74.35) (width 0.15) (layer "F.Cu") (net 3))
 (segment (start 108.830905 77.665346) (end 108.704553 77.538994) (width 0.15) (layer "F.Cu") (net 3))
 (segment (start 105.175 73.075) (end 106.029296 72.220704) (width 0.15) (layer "F.Cu") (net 3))
 (segment (start 104.394 72.339076) (end 103.659905 73.073171) (width 0.15) (layer "F.Cu") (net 3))
 (segment (start 107.137822 77.538994) (end 107.039898 77.44107) (width 0.15) (layer "F.Cu") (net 3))
 (segment (start 103.925282 78.019406) (end 105.197406 78.019406) (width 0.25) (layer "F.Cu") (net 1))
 (segment (start 107.801898 78.041131) (end 107.539897 78.303132) (width 0.15) (layer "F.Cu") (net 1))
 (segment (start 107.442 78.74) (end 107.539897 78.642103) (width 0.25) (layer "F.Cu") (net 1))
 (segment (start 107.801898 77.791132) (end 107.801898 78.041131) (width 0.15) (layer "F.Cu") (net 1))
 (segment (start 105.918 78.74) (end 107.442 78.74) (width 0.25) (layer "F.Cu") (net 1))
 (segment (start 104.075 76.670073) (end 104.09078 76.685853) (width 0.25) (layer "F.Cu") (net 1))
 (segment (start 105.197406 78.019406) (end 105.255263 77.961549) (width 0.25) (layer "F.Cu") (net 1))
 (segment (start 104.075 75.75) (end 104.075 76.670073) (width 0.25) (layer "F.Cu") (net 1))
 (segment (start 109.5 75.5) (end 109.5 77.952) (width 0.25) (layer "F.Cu") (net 1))
 (segment (start 109.148868 78.303132) (end 107.539897 78.303132) (width 0.25) (layer "F.Cu") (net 1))
 (segment (start 105.255263 77.961549) (end 105.255263 77.533434) (width 0.25) (layer "F.Cu") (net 1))
 (segment (start 107.539897 78.642103) (end 107.539897 78.303132) (width 0.25) (layer "F.Cu") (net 1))
 (segment (start 104.09078 76.685853) (end 104.09078 77.853908) (width 0.25) (layer "F.Cu") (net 1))
 (segment (start 105.197406 78.019406) (end 105.918 78.74) (width 0.25) (layer "F.Cu") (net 1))
 (segment (start 109.5 77.952) (end 109.148868 78.303132) (width 0.25) (layer "F.Cu") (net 1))
 (segment (start 104.09078 77.853908) (end 103.925282 78.019406) (width 0.25) (layer "F.Cu") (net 1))
 (segment (start 108.9 76.636251) (end 108.830905 76.705346) (width 0.25) (layer "F.Cu") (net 2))
 (segment (start 108.9 75.5) (end 108.9 76.636251) (width 0.25) (layer "F.Cu") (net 2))
 (segment (start 104.648 72.429987) (end 105.281186 71.796801) (width 0.25) (layer "F.Cu") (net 10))
 (segment (start 104.648 73.223) (end 104.648 72.429987) (width 0.25) (layer "F.Cu") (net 10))
 (segment (start 104.648 73.223) (end 105.175 73.75) (width 0.25) (layer "F.Cu") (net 10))
 (segment (start 105.9 73.2) (end 105.9 72.788596) (width 0.25) (layer "F.Cu") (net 19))
 (segment (start 105.9 72.788596) (end 107.024773 71.663823) (width 0.25) (layer "F.Cu") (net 19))
 (segment (start 108.993071 74.809519) (end 108.993071 73.902867) (width 0.15) (layer "F.Cu") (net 4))
 (segment (start 107.801898 77.291132) (end 107.801898 76.856102) (width 0.15) (layer "F.Cu") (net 4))
 (segment (start 106.931 72.644) (end 108.204 72.644) (width 0.25) (layer "F.Cu") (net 4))
 (segment (start 108.60663 76.05137) (end 108.60663 75.19596) (width 0.15) (layer "F.Cu") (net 4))
 (segment (start 108.591644 73.50144) (end 108.591644 72.777644) (width 0.15) (layer "F.Cu") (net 4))
 (segment (start 108.712 72.657288) (end 108.712 72.136) (width 0.15) (layer "F.Cu") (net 4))
 (segment (start 108.712 72.136) (end 108.712 71.628) (width 0.15) (layer "F.Cu") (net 4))
 (segment (start 107.801898 76.856102) (end 108.60663 76.05137) (width 0.15) (layer "F.Cu") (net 4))
 (segment (start 108.60663 75.19596) (end 108.993071 74.809519) (width 0.15) (layer "F.Cu") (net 4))
 (segment (start 108.204 72.644) (end 108.712 72.136) (width 0.25) (layer "F.Cu") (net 4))
 (segment (start 108.591644 72.777644) (end 108.712 72.657288) (width 0.15) (layer "F.Cu") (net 4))
 (segment (start 106.5 73.075) (end 106.931 72.644) (width 0.25) (layer "F.Cu") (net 4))
 (segment (start 106.5 73.2) (end 106.5 73.075) (width 0.25) (layer "F.Cu") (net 4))
 (segment (start 108.993071 73.902867) (end 108.591644 73.50144) (width 0.15) (layer "F.Cu") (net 4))
 (segment (start 103.159905 72.155828) (end 103.159905 73.073171) (width 0.25) (layer "F.Cu") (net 9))
 (segment (start 103.647128 71.668605) (end 103.159905 72.155828) (width 0.25) (layer "F.Cu") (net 9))
 (segment (start 105.175 74.35) (end 105.05 74.35) (width 0.25) (layer "F.Cu") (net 20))
 (segment (start 104.159905 73.459905) (end 104.159905 73.073171) (width 0.25) (layer "F.Cu") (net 20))
 (segment (start 105.05 74.35) (end 104.159905 73.459905) (width 0.25) (layer "F.Cu") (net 20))
 (segment (start 109.511837 72.588236) (end 109.509684 72.590389) (width 0.15) (layer "F.Cu") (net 15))
 (segment (start 109.671093 72.588236) (end 109.511837 72.588236) (width 0.15) (layer "F.Cu") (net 15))
 (segment (start 109.5 72.600073) (end 109.5 73.2) (width 0.15) (layer "F.Cu") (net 15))
 (segment (start 109.509684 72.590389) (end 109.5 72.600073) (width 0.15) (layer "F.Cu") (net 15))
 (segment (start 107.7 75.942) (end 107.7 75.5) (width 0.25) (layer "F.Cu") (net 5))
 (segment (start 107.039898 76.779132) (end 107.039898 76.602102) (width 0.25) (layer "F.Cu") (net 5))
 (segment (start 107.039898 76.602102) (end 107.7 75.942) (width 0.25) (layer "F.Cu") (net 5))
 (segment (start 105.9 75.5) (end 105.9 76.913234) (width 0.25) (layer "F.Cu") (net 7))
 (segment (start 105.9 76.913234) (end 106.277898 77.291132) (width 0.25) (layer "F.Cu") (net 7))
 (segment (start 106.539899 76.779132) (end 106.539899 76.340101) (width 0.25) (layer "F.Cu") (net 6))
 (segment (start 107.1 75.78) (end 107.1 75.5) (width 0.25) (layer "F.Cu") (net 6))
 (segment (start 106.539899 76.340101) (end 107.1 75.78) (width 0.25) (layer "F.Cu") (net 6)))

